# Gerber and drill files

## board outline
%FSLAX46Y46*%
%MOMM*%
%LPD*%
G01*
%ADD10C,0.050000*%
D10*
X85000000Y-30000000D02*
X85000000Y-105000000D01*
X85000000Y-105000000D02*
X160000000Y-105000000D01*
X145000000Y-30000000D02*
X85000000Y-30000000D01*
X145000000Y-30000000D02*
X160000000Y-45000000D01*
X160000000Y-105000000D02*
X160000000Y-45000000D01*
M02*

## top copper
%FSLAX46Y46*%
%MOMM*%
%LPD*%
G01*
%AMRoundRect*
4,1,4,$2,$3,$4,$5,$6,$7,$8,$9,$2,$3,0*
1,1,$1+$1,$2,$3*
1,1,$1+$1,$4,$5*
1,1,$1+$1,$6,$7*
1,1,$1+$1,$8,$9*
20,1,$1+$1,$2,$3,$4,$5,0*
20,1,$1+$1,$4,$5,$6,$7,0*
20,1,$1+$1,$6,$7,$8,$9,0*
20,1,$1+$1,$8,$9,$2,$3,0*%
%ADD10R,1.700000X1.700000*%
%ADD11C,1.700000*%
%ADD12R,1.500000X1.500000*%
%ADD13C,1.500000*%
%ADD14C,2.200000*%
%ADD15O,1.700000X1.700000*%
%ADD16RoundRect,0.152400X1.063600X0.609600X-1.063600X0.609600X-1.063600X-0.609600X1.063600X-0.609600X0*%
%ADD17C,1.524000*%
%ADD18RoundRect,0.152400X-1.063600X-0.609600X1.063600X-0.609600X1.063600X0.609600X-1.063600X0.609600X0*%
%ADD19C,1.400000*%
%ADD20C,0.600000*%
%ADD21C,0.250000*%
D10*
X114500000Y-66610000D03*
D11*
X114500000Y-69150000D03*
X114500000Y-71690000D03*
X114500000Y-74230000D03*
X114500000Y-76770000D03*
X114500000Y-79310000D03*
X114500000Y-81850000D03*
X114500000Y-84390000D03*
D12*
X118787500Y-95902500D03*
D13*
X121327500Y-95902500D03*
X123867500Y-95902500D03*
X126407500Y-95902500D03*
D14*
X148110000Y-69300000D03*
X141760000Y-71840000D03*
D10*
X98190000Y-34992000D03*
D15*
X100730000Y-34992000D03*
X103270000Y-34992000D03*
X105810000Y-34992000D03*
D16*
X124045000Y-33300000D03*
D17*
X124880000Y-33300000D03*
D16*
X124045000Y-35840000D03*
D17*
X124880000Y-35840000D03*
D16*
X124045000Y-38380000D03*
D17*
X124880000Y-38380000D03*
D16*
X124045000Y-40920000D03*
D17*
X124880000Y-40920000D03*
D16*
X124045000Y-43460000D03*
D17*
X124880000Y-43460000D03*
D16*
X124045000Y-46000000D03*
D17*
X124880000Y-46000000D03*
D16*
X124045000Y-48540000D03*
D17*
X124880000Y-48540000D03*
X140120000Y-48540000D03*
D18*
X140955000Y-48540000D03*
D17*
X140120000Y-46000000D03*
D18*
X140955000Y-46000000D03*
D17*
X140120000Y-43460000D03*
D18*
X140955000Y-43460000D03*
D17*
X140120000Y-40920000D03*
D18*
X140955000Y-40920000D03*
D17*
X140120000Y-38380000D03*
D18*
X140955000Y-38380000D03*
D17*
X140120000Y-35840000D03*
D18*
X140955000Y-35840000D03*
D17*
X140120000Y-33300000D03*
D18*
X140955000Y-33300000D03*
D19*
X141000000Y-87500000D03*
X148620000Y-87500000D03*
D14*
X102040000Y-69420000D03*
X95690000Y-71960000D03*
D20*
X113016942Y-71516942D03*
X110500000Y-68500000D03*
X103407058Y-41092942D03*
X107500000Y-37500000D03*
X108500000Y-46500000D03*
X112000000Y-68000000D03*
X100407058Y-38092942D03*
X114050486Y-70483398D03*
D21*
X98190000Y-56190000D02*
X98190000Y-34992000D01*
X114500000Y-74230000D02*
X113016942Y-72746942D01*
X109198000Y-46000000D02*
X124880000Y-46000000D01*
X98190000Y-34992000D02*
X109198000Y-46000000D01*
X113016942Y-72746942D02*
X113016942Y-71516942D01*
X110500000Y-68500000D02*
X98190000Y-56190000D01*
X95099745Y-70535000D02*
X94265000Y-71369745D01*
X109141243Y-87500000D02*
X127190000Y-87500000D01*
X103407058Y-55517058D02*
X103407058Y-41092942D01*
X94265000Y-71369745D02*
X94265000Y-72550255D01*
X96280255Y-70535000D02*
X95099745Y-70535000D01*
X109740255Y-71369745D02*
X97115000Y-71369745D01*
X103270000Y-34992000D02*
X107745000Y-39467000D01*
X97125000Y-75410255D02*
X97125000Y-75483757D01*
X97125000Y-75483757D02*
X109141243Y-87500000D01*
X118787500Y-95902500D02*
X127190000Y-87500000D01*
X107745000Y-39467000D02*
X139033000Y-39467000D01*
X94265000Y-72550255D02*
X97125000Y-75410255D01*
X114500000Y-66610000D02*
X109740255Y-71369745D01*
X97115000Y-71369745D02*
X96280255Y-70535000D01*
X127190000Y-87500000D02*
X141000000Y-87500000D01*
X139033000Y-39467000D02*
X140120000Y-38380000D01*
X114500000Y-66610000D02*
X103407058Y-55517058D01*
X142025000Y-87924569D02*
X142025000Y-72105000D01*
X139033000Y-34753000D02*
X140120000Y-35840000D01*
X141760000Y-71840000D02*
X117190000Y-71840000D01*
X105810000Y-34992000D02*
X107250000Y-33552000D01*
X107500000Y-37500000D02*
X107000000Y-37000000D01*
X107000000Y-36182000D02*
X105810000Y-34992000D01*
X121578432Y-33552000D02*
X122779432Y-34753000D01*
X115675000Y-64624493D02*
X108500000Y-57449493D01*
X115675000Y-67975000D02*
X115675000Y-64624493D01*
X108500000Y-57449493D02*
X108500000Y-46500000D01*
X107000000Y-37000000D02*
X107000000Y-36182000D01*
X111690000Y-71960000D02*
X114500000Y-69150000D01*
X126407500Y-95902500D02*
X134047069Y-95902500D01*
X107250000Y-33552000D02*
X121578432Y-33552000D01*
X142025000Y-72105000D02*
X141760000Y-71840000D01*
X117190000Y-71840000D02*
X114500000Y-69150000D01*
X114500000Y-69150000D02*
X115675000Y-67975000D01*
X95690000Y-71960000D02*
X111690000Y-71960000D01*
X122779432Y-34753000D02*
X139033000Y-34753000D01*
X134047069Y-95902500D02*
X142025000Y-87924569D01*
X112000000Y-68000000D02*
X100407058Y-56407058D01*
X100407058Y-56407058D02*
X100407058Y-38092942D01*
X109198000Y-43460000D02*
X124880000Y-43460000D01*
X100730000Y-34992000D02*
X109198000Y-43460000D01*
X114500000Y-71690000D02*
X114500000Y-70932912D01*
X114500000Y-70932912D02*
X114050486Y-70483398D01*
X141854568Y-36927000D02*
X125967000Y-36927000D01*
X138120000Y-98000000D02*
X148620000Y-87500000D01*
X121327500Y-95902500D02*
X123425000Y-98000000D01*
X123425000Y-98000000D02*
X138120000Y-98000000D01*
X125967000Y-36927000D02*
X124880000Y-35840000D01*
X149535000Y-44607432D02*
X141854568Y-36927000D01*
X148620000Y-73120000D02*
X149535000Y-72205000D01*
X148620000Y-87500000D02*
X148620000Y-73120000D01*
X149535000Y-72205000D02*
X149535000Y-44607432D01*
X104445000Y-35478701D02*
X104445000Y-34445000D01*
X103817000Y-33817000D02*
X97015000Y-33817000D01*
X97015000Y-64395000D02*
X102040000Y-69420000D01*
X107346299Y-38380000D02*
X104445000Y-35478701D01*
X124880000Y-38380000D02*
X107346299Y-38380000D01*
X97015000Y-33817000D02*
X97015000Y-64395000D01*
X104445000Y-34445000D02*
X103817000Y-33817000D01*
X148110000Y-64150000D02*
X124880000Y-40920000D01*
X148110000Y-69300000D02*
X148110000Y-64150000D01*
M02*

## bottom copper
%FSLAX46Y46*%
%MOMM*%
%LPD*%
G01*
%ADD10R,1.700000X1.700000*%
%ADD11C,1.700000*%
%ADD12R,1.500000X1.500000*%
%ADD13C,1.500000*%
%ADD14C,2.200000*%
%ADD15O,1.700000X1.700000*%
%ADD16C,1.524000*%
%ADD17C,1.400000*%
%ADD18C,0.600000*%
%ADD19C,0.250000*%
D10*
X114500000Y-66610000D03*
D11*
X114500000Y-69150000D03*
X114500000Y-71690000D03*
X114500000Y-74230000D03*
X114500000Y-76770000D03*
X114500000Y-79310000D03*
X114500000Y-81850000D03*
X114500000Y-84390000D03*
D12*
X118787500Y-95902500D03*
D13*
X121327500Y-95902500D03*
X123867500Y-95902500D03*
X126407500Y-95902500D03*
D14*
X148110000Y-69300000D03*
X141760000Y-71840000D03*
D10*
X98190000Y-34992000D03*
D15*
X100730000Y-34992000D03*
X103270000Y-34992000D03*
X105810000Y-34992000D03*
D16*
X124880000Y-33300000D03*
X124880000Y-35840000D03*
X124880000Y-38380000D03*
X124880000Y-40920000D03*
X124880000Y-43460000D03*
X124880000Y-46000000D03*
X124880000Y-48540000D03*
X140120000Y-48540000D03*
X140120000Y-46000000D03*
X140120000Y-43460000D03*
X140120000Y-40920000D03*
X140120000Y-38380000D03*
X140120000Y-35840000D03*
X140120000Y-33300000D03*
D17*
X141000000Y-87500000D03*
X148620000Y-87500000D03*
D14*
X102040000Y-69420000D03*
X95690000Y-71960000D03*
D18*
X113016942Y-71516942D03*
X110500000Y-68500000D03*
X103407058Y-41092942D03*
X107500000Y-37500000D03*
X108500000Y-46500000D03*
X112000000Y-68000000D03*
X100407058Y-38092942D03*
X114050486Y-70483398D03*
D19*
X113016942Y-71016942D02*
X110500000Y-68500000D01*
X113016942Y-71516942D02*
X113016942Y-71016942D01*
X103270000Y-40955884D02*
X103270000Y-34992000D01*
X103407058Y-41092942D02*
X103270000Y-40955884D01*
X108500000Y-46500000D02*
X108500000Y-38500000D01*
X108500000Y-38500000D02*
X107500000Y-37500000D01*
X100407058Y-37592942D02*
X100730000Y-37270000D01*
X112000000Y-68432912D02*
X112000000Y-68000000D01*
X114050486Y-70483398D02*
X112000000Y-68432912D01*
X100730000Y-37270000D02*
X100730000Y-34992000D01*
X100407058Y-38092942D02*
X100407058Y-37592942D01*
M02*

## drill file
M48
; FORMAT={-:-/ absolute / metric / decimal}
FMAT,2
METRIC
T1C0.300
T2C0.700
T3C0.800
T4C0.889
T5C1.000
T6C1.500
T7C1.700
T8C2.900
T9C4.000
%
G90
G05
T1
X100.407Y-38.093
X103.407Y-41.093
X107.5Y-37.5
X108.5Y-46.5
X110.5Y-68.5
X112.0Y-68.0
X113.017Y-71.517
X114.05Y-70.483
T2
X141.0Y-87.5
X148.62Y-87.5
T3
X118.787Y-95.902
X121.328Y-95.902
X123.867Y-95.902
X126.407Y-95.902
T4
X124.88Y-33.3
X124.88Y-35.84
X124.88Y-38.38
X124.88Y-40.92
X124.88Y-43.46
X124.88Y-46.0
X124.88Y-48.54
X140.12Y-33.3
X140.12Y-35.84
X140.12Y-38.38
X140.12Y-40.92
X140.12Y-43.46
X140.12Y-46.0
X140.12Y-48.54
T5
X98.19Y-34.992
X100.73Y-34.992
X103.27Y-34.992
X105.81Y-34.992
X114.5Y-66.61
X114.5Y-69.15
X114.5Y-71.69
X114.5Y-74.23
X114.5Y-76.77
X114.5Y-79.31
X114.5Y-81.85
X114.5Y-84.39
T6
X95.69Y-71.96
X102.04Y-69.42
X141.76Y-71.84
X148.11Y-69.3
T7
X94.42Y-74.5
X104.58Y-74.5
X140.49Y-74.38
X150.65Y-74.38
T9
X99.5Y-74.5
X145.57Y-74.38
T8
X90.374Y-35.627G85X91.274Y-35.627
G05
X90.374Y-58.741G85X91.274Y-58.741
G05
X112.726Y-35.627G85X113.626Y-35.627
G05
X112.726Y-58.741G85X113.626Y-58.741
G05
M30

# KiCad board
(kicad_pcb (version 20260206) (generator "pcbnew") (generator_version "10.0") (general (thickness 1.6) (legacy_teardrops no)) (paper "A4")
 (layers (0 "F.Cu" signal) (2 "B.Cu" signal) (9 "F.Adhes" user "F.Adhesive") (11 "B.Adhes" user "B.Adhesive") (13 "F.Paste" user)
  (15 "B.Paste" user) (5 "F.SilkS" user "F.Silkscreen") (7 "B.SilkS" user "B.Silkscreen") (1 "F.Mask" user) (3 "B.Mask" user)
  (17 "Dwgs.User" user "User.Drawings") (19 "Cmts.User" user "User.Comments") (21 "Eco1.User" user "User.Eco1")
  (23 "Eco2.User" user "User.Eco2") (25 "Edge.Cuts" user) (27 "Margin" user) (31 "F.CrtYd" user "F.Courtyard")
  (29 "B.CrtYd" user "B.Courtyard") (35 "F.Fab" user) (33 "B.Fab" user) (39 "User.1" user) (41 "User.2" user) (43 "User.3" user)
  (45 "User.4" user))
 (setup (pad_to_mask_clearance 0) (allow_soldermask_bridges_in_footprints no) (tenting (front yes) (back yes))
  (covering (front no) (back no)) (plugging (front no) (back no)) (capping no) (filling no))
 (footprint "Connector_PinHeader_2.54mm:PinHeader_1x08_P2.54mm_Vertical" (layer "F.Cu") (at 114.5 66.61)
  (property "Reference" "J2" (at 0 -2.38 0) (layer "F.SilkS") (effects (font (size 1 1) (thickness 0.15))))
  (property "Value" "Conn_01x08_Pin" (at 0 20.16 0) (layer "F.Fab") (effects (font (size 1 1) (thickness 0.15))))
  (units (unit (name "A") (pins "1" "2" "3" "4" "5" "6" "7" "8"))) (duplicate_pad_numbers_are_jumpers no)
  (pad "1" thru_hole rect (at 0 0) (size 1.7 1.7) (drill 1) (layers "*.Cu" "*.Mask") (remove_unused_layers no) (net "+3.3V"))
  (pad "2" thru_hole circle (at 0 2.54) (size 1.7 1.7) (drill 1) (layers "*.Cu" "*.Mask") (remove_unused_layers no) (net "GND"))
  (pad "3" thru_hole circle (at 0 5.08) (size 1.7 1.7) (drill 1) (layers "*.Cu" "*.Mask") (remove_unused_layers no) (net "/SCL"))
  (pad "4" thru_hole circle (at 0 7.62) (size 1.7 1.7) (drill 1) (layers "*.Cu" "*.Mask") (remove_unused_layers no) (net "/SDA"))
  (pad "5" thru_hole circle (at 0 10.16) (size 1.7 1.7) (drill 1) (layers "*.Cu" "*.Mask") (remove_unused_layers no)
   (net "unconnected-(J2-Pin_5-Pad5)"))
  (pad "6" thru_hole circle (at 0 12.7) (size 1.7 1.7) (drill 1) (layers "*.Cu" "*.Mask") (remove_unused_layers no)
   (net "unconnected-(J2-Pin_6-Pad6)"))
  (pad "7" thru_hole circle (at 0 15.24) (size 1.7 1.7) (drill 1) (layers "*.Cu" "*.Mask") (remove_unused_layers no)
   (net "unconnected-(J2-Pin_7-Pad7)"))
  (pad "8" thru_hole circle (at 0 17.78) (size 1.7 1.7) (drill 1) (layers "*.Cu" "*.Mask") (remove_unused_layers no)
   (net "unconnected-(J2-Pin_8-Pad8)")))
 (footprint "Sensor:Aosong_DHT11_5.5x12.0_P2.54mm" (layer "F.Cu") (at 118.7875 95.9025 90)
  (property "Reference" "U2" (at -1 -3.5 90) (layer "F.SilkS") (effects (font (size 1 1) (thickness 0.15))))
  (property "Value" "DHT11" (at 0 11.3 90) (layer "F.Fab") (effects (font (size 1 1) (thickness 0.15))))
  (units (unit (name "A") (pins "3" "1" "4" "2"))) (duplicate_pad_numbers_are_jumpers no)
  (pad "1" thru_hole rect (at 0 0 90) (size 1.5 1.5) (drill 0.8) (layers "*.Cu" "*.Mask") (remove_unused_layers no) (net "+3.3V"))
  (pad "2" thru_hole circle (at 0 2.54 90) (size 1.5 1.5) (drill 0.8) (layers "*.Cu" "*.Mask") (remove_unused_layers no) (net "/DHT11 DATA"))
  (pad "3" thru_hole circle (at 0 5.08 90) (size 1.5 1.5) (drill 0.8) (layers "*.Cu" "*.Mask") (remove_unused_layers no)
   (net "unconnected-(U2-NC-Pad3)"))
  (pad "4" thru_hole circle (at 0 7.62 90) (size 1.5 1.5) (drill 0.8) (layers "*.Cu" "*.Mask") (remove_unused_layers no) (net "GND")))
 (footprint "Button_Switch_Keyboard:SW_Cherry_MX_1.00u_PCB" (layer "F.Cu") (at 148.11 69.3)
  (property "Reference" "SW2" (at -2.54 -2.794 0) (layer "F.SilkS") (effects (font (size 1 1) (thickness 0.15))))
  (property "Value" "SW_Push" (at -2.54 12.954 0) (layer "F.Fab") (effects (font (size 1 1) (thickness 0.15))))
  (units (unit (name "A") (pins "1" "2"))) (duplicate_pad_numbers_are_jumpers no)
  (pad "" np_thru_hole circle (at -7.62 5.08) (size 1.7 1.7) (drill 1.7) (layers "*.Cu" "*.Mask"))
  (pad "" np_thru_hole circle (at -2.54 5.08) (size 4 4) (drill 4) (layers "*.Cu" "*.Mask"))
  (pad "" np_thru_hole circle (at 2.54 5.08) (size 1.7 1.7) (drill 1.7) (layers "*.Cu" "*.Mask"))
  (pad "1" thru_hole circle (at 0 0) (size 2.2 2.2) (drill 1.5) (layers "*.Cu" "*.Mask") (remove_unused_layers no) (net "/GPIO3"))
  (pad "2" thru_hole circle (at -6.35 2.54) (size 2.2 2.2) (drill 1.5) (layers "*.Cu" "*.Mask") (remove_unused_layers no) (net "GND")))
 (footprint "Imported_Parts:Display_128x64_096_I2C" (layer "F.Cu") (at 102 34.992)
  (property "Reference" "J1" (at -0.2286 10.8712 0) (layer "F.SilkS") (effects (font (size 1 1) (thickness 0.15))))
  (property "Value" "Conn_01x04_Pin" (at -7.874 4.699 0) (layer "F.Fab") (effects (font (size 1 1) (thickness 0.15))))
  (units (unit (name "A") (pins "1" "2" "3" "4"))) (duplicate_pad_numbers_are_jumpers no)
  (pad "" np_thru_hole oval (at -11.176 0.635) (size 3.8 2.9) (drill oval 3.8 2.9) (layers "*.Cu" "*.Mask"))
  (pad "" np_thru_hole oval (at -11.176 23.749) (size 3.8 2.9) (drill oval 3.8 2.9) (layers "*.Cu" "*.Mask"))
  (pad "" np_thru_hole oval (at 11.176 0.635) (size 3.8 2.9) (drill oval 3.8 2.9) (layers "*.Cu" "*.Mask"))
  (pad "" np_thru_hole oval (at 11.176 23.749) (size 3.8 2.9) (drill oval 3.8 2.9) (layers "*.Cu" "*.Mask"))
  (pad "1" thru_hole rect (at -3.81 0 90) (size 1.7 1.7) (drill 1) (layers "*.Cu" "*.Mask") (remove_unused_layers no) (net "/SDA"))
  (pad "2" thru_hole oval (at -1.27 0 90) (size 1.7 1.7) (drill 1) (layers "*.Cu" "*.Mask") (remove_unused_layers no) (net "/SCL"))
  (pad "3" thru_hole oval (at 1.27 0 90) (size 1.7 1.7) (drill 1) (layers "*.Cu" "*.Mask") (remove_unused_layers no) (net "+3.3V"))
  (pad "4" thru_hole oval (at 3.81 0 90) (size 1.7 1.7) (drill 1) (layers "*.Cu" "*.Mask") (remove_unused_layers no) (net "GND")))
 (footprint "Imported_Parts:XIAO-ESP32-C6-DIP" (layer "F.Cu") (at 132.5 40.92 90)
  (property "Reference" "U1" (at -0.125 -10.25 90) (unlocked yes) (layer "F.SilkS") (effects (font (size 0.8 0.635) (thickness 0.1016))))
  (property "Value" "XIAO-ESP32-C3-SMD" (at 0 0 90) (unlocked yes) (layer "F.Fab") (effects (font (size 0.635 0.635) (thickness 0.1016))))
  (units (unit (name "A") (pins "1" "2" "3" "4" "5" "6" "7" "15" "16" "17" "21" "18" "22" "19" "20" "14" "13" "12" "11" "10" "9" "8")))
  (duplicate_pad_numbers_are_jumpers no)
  (pad "1" smd roundrect (at 7.62 -8.455 180) (size 2.432 1.524) (layers "F.Cu" "F.Mask") (roundrect_rratio 0.1)
   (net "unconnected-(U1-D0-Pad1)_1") (thermal_bridge_angle 45))
  (pad "1" thru_hole circle (at 7.62 -7.62 180) (size 1.524 1.524) (drill 0.889) (layers "*.Cu" "*.Mask") (remove_unused_layers no)
   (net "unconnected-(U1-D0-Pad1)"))
  (pad "2" smd roundrect (at 5.08 -8.455 180) (size 2.432 1.524) (layers "F.Cu" "F.Mask") (roundrect_rratio 0.1) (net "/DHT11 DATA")
   (thermal_bridge_angle 45))
  (pad "2" thru_hole circle (at 5.08 -7.62 180) (size 1.524 1.524) (drill 0.889) (layers "*.Cu" "*.Mask") (remove_unused_layers no)
   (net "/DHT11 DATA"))
  (pad "3" smd roundrect (at 2.54 -8.455 180) (size 2.432 1.524) (layers "F.Cu" "F.Mask") (roundrect_rratio 0.1) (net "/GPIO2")
   (thermal_bridge_angle 45))
  (pad "3" thru_hole circle (at 2.54 -7.62 180) (size 1.524 1.524) (drill 0.889) (layers "*.Cu" "*.Mask") (remove_unused_layers no)
   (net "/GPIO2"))
  (pad "4" smd roundrect (at 0 -8.455 180) (size 2.432 1.524) (layers "F.Cu" "F.Mask") (roundrect_rratio 0.1) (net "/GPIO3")
   (thermal_bridge_angle 45))
  (pad "4" thru_hole circle (at 0 -7.62 180) (size 1.524 1.524) (drill 0.889) (layers "*.Cu" "*.Mask") (remove_unused_layers no)
   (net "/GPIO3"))
  (pad "5" smd roundrect (at -2.54 -8.455 180) (size 2.432 1.524) (layers "F.Cu" "F.Mask") (roundrect_rratio 0.1) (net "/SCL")
   (thermal_bridge_angle 45))
  (pad "5" thru_hole circle (at -2.54 -7.62 180) (size 1.524 1.524) (drill 0.889) (layers "*.Cu" "*.Mask") (remove_unused_layers no)
   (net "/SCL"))
  (pad "6" smd roundrect (at -5.08 -8.455 180) (size 2.432 1.524) (layers "F.Cu" "F.Mask") (roundrect_rratio 0.1) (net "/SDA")
   (thermal_bridge_angle 45))
  (pad "6" thru_hole circle (at -5.08 -7.62 180) (size 1.524 1.524) (drill 0.889) (layers "*.Cu" "*.Mask") (remove_unused_layers no)
   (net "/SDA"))
  (pad "7" smd roundrect (at -7.62 -8.455 180) (size 2.432 1.524) (layers "F.Cu" "F.Mask") (roundrect_rratio 0.1)
   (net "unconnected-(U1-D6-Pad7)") (thermal_bridge_angle 45))
  (pad "7" thru_hole circle (at -7.62 -7.62 180) (size 1.524 1.524) (drill 0.889) (layers "*.Cu" "*.Mask") (remove_unused_layers no)
   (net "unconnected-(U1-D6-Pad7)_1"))
  (pad "8" thru_hole circle (at -7.62 7.62) (size 1.524 1.524) (drill 0.889) (layers "*.Cu" "*.Mask") (remove_unused_layers no)
   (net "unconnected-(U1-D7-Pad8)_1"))
  (pad "8" smd roundrect (at -7.62 8.455) (size 2.432 1.524) (layers "F.Cu" "F.Mask") (roundrect_rratio 0.1)
   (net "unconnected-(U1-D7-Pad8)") (thermal_bridge_angle 45))
  (pad "9" thru_hole circle (at -5.08 7.62) (size 1.524 1.524) (drill 0.889) (layers "*.Cu" "*.Mask") (remove_unused_layers no)
   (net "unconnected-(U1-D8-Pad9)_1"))
  (pad "9" smd roundrect (at -5.08 8.455) (size 2.432 1.524) (layers "F.Cu" "F.Mask") (roundrect_rratio 0.1)
   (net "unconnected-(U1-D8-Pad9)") (thermal_bridge_angle 45))
  (pad "10" thru_hole circle (at -2.54 7.62) (size 1.524 1.524) (drill 0.889) (layers "*.Cu" "*.Mask") (remove_unused_layers no)
   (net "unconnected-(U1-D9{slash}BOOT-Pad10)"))
  (pad "10" smd roundrect (at -2.54 8.455) (size 2.432 1.524) (layers "F.Cu" "F.Mask") (roundrect_rratio 0.1)
   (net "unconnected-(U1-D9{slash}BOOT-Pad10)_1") (thermal_bridge_angle 45))
  (pad "11" thru_hole circle (at 0 7.62) (size 1.524 1.524) (drill 0.889) (layers "*.Cu" "*.Mask") (remove_unused_layers no)
   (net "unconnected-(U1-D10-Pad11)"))
  (pad "11" smd roundrect (at 0 8.455) (size 2.432 1.524) (layers "F.Cu" "F.Mask") (roundrect_rratio 0.1)
   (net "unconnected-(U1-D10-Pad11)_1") (thermal_bridge_angle 45))
  (pad "12" thru_hole circle (at 2.54 7.62) (size 1.524 1.524) (drill 0.889) (layers "*.Cu" "*.Mask") (remove_unused_layers no)
   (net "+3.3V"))
  (pad "12" smd roundrect (at 2.54 8.455) (size 2.432 1.524) (layers "F.Cu" "F.Mask") (roundrect_rratio 0.1) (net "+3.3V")
   (thermal_bridge_angle 45))
  (pad "13" thru_hole circle (at 5.08 7.62) (size 1.524 1.524) (drill 0.889) (layers "*.Cu" "*.Mask") (remove_unused_layers no) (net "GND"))
  (pad "13" smd roundrect (at 5.08 8.455) (size 2.432 1.524) (layers "F.Cu" "F.Mask") (roundrect_rratio 0.1) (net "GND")
   (thermal_bridge_angle 45))
  (pad "14" thru_hole circle (at 7.62 7.62) (size 1.524 1.524) (drill 0.889) (layers "*.Cu" "*.Mask") (remove_unused_layers no) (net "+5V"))
  (pad "14" smd roundrect (at 7.62 8.455) (size 2.432 1.524) (layers "F.Cu" "F.Mask") (roundrect_rratio 0.1) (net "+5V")
   (thermal_bridge_angle 45)))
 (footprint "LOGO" (layer "F.Cu") (at 101 94)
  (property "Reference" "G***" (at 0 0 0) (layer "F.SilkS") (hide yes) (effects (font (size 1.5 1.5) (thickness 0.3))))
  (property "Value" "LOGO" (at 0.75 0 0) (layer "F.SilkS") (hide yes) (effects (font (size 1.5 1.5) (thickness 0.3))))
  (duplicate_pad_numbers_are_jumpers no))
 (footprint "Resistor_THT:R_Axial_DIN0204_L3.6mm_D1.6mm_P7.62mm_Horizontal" (layer "F.Cu") (at 141 87.5)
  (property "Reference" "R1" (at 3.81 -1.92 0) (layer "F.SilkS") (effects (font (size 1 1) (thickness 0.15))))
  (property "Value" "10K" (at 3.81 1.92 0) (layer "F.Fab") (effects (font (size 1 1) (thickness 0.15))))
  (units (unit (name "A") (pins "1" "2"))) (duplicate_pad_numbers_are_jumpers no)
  (pad "1" thru_hole circle (at 0 0) (size 1.4 1.4) (drill 0.7) (layers "*.Cu" "*.Mask") (remove_unused_layers no) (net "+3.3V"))
  (pad "2" thru_hole circle (at 7.62 0) (size 1.4 1.4) (drill 0.7) (layers "*.Cu" "*.Mask") (remove_unused_layers no) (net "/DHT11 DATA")))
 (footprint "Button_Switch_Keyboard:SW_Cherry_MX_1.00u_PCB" (layer "F.Cu") (at 102.04 69.42)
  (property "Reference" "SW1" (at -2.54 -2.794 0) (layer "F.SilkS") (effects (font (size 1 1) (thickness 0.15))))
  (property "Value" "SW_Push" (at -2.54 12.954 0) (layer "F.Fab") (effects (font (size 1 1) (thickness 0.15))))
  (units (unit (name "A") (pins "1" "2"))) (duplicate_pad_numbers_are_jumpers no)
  (pad "" np_thru_hole circle (at -7.62 5.08) (size 1.7 1.7) (drill 1.7) (layers "*.Cu" "*.Mask"))
  (pad "" np_thru_hole circle (at -2.54 5.08) (size 4 4) (drill 4) (layers "*.Cu" "*.Mask"))
  (pad "" np_thru_hole circle (at 2.54 5.08) (size 1.7 1.7) (drill 1.7) (layers "*.Cu" "*.Mask"))
  (pad "1" thru_hole circle (at 0 0) (size 2.2 2.2) (drill 1.5) (layers "*.Cu" "*.Mask") (remove_unused_layers no) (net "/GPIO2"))
  (pad "2" thru_hole circle (at -6.35 2.54) (size 2.2 2.2) (drill 1.5) (layers "*.Cu" "*.Mask") (remove_unused_layers no) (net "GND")))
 (gr_line (start 85 30) (end 85 105) (stroke (width 0.05) (type default)) (layer "Edge.Cuts"))
 (gr_line (start 85 105) (end 160 105) (stroke (width 0.05) (type default)) (layer "Edge.Cuts"))
 (gr_line (start 145 30) (end 85 30) (stroke (width 0.05) (type default)) (layer "Edge.Cuts"))
 (gr_line (start 145 30) (end 160 45) (stroke (width 0.05) (type default)) (layer "Edge.Cuts"))
 (gr_line (start 160 105) (end 160 45) (stroke (width 0.05) (type default)) (layer "Edge.Cuts"))
 (segment (start 98.19 56.19) (end 98.19 34.992) (width 0.25) (layer "F.Cu") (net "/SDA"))
 (segment (start 114.5 74.23) (end 113.016942 72.746942) (width 0.25) (layer "F.Cu") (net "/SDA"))
 (segment (start 109.198 46) (end 124.88 46) (width 0.25) (layer "F.Cu") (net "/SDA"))
 (segment (start 98.19 34.992) (end 109.198 46) (width 0.25) (layer "F.Cu") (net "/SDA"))
 (segment (start 113.016942 72.746942) (end 113.016942 71.516942) (width 0.25) (layer "F.Cu") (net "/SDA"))
 (segment (start 110.5 68.5) (end 98.19 56.19) (width 0.25) (layer "F.Cu") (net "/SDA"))
 (via (at 113.016942 71.516942) (size 0.6) (drill 0.3) (layers "F.Cu" "B.Cu") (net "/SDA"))
 (via (at 110.5 68.5) (size 0.6) (drill 0.3) (layers "F.Cu" "B.Cu") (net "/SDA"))
 (segment (start 113.016942 71.016942) (end 110.5 68.5) (width 0.25) (layer "B.Cu") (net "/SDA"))
 (segment (start 113.016942 71.516942) (end 113.016942 71.016942) (width 0.25) (layer "B.Cu") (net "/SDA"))
 (segment (start 95.099745 70.535) (end 94.265 71.369745) (width 0.25) (layer "F.Cu") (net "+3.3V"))
 (segment (start 109.141243 87.5) (end 127.19 87.5) (width 0.25) (layer "F.Cu") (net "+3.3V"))
 (segment (start 103.407058 55.517058) (end 103.407058 41.092942) (width 0.25) (layer "F.Cu") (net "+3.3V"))
 (segment (start 94.265 71.369745) (end 94.265 72.550255) (width 0.25) (layer "F.Cu") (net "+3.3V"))
 (segment (start 96.280255 70.535) (end 95.099745 70.535) (width 0.25) (layer "F.Cu") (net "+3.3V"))
 (segment (start 109.740255 71.369745) (end 97.115 71.369745) (width 0.25) (layer "F.Cu") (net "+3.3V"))
 (segment (start 103.27 34.992) (end 107.745 39.467) (width 0.25) (layer "F.Cu") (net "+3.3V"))
 (segment (start 97.125 75.410255) (end 97.125 75.483757) (width 0.25) (layer "F.Cu") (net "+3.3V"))
 (segment (start 97.125 75.483757) (end 109.141243 87.5) (width 0.25) (layer "F.Cu") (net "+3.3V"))
 (segment (start 118.7875 95.9025) (end 127.19 87.5) (width 0.25) (layer "F.Cu") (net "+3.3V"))
 (segment (start 107.745 39.467) (end 139.033 39.467) (width 0.25) (layer "F.Cu") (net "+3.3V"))
 (segment (start 94.265 72.550255) (end 97.125 75.410255) (width 0.25) (layer "F.Cu") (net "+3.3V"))
 (segment (start 114.5 66.61) (end 109.740255 71.369745) (width 0.25) (layer "F.Cu") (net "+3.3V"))
 (segment (start 97.115 71.369745) (end 96.280255 70.535) (width 0.25) (layer "F.Cu") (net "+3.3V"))
 (segment (start 127.19 87.5) (end 141 87.5) (width 0.25) (layer "F.Cu") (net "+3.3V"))
 (segment (start 139.033 39.467) (end 140.12 38.38) (width 0.25) (layer "F.Cu") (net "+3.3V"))
 (segment (start 114.5 66.61) (end 103.407058 55.517058) (width 0.25) (layer "F.Cu") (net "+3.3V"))
 (via (at 103.407058 41.092942) (size 0.6) (drill 0.3) (layers "F.Cu" "B.Cu") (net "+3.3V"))
 (segment (start 103.27 40.955884) (end 103.27 34.992) (width 0.25) (layer "B.Cu") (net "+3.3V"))
 (segment (start 103.407058 41.092942) (end 103.27 40.955884) (width 0.25) (layer "B.Cu") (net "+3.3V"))
 (segment (start 142.025 87.924569) (end 142.025 72.105) (width 0.25) (layer "F.Cu") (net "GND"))
 (segment (start 139.033 34.753) (end 140.12 35.84) (width 0.25) (layer "F.Cu") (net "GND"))
 (segment (start 141.76 71.84) (end 117.19 71.84) (width 0.25) (layer "F.Cu") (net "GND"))
 (segment (start 105.81 34.992) (end 107.25 33.552) (width 0.25) (layer "F.Cu") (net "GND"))
 (segment (start 107.5 37.5) (end 107 37) (width 0.25) (layer "F.Cu") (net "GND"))
 (segment (start 107 36.182) (end 105.81 34.992) (width 0.25) (layer "F.Cu") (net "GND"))
 (segment (start 121.578432 33.552) (end 122.779432 34.753) (width 0.25) (layer "F.Cu") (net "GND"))
 (segment (start 115.675 64.624493) (end 108.5 57.449493) (width 0.25) (layer "F.Cu") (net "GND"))
 (segment (start 115.675 67.975) (end 115.675 64.624493) (width 0.25) (layer "F.Cu") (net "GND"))
 (segment (start 108.5 57.449493) (end 108.5 46.5) (width 0.25) (layer "F.Cu") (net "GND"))
 (segment (start 107 37) (end 107 36.182) (width 0.25) (layer "F.Cu") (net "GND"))
 (segment (start 111.69 71.96) (end 114.5 69.15) (width 0.25) (layer "F.Cu") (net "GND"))
 (segment (start 126.4075 95.9025) (end 134.047069 95.9025) (width 0.25) (layer "F.Cu") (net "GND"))
 (segment (start 107.25 33.552) (end 121.578432 33.552) (width 0.25) (layer "F.Cu") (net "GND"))
 (segment (start 142.025 72.105) (end 141.76 71.84) (width 0.25) (layer "F.Cu") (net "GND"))
 (segment (start 117.19 71.84) (end 114.5 69.15) (width 0.25) (layer "F.Cu") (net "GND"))
 (segment (start 114.5 69.15) (end 115.675 67.975) (width 0.25) (layer "F.Cu") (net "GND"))
 (segment (start 95.69 71.96) (end 111.69 71.96) (width 0.25) (layer "F.Cu") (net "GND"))
 (segment (start 122.779432 34.753) (end 139.033 34.753) (width 0.25) (layer "F.Cu") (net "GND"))
 (segment (start 134.047069 95.9025) (end 142.025 87.924569) (width 0.25) (layer "F.Cu") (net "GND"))
 (via (at 107.5 37.5) (size 0.6) (drill 0.3) (layers "F.Cu" "B.Cu") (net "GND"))
 (via (at 108.5 46.5) (size 0.6) (drill 0.3) (layers "F.Cu" "B.Cu") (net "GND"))
 (segment (start 108.5 46.5) (end 108.5 38.5) (width 0.25) (layer "B.Cu") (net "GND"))
 (segment (start 108.5 38.5) (end 107.5 37.5) (width 0.25) (layer "B.Cu") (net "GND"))
 (segment (start 112 68) (end 100.407058 56.407058) (width 0.25) (layer "F.Cu") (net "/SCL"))
 (segment (start 100.407058 56.407058) (end 100.407058 38.092942) (width 0.25) (layer "F.Cu") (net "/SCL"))
 (segment (start 109.198 43.46) (end 124.88 43.46) (width 0.25) (layer "F.Cu") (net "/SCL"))
 (segment (start 100.73 34.992) (end 109.198 43.46) (width 0.25) (layer "F.Cu") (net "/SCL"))
 (segment (start 114.5 71.69) (end 114.5 70.932912) (width 0.25) (layer "F.Cu") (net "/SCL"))
 (segment (start 114.5 70.932912) (end 114.050486 70.483398) (width 0.25) (layer "F.Cu") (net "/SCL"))
 (via (at 112 68) (size 0.6) (drill 0.3) (layers "F.Cu" "B.Cu") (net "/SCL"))
 (via (at 100.407058 38.092942) (size 0.6) (drill 0.3) (layers "F.Cu" "B.Cu") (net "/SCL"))
 (via (at 114.050486 70.483398) (size 0.6) (drill 0.3) (layers "F.Cu" "B.Cu") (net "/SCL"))
 (segment (start 100.407058 37.592942) (end 100.73 37.27) (width 0.25) (layer "B.Cu") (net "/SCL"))
 (segment (start 112 68.432912) (end 112 68) (width 0.25) (layer "B.Cu") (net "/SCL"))
 (segment (start 114.050486 70.483398) (end 112 68.432912) (width 0.25) (layer "B.Cu") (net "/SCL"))
 (segment (start 100.73 37.27) (end 100.73 34.992) (width 0.25) (layer "B.Cu") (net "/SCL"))
 (segment (start 100.407058 38.092942) (end 100.407058 37.592942) (width 0.25) (layer "B.Cu") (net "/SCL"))
 (segment (start 141.854568 36.927) (end 125.967 36.927) (width 0.25) (layer "F.Cu") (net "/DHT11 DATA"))
 (segment (start 138.12 98) (end 148.62 87.5) (width 0.25) (layer "F.Cu") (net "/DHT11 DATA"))
 (segment (start 121.3275 95.9025) (end 123.425 98) (width 0.25) (layer "F.Cu") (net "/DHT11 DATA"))
 (segment (start 123.425 98) (end 138.12 98) (width 0.25) (layer "F.Cu") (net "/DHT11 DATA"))
 (segment (start 125.967 36.927) (end 124.88 35.84) (width 0.25) (layer "F.Cu") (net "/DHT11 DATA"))
 (segment (start 149.535 44.607432) (end 141.854568 36.927) (width 0.25) (layer "F.Cu") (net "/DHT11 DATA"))
 (segment (start 148.62 73.12) (end 149.535 72.205) (width 0.25) (layer "F.Cu") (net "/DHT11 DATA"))
 (segment (start 148.62 87.5) (end 148.62 73.12) (width 0.25) (layer "F.Cu") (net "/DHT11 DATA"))
 (segment (start 149.535 72.205) (end 149.535 44.607432) (width 0.25) (layer "F.Cu") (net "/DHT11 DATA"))
 (segment (start 104.445 35.478701) (end 104.445 34.445) (width 0.25) (layer "F.Cu") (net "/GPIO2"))
 (segment (start 103.817 33.817) (end 97.015 33.817) (width 0.25) (layer "F.Cu") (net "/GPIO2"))
 (segment (start 97.015 64.395) (end 102.04 69.42) (width 0.25) (layer "F.Cu") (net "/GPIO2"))
 (segment (start 107.346299 38.38) (end 104.445 35.478701) (width 0.25) (layer "F.Cu") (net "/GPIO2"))
 (segment (start 124.88 38.38) (end 107.346299 38.38) (width 0.25) (layer "F.Cu") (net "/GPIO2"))
 (segment (start 97.015 33.817) (end 97.015 64.395) (width 0.25) (layer "F.Cu") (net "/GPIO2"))
 (segment (start 104.445 34.445) (end 103.817 33.817) (width 0.25) (layer "F.Cu") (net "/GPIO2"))
 (segment (start 148.11 64.15) (end 124.88 40.92) (width 0.25) (layer "F.Cu") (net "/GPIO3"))
 (segment (start 148.11 69.3) (end 148.11 64.15) (width 0.25) (layer "F.Cu") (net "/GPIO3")))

